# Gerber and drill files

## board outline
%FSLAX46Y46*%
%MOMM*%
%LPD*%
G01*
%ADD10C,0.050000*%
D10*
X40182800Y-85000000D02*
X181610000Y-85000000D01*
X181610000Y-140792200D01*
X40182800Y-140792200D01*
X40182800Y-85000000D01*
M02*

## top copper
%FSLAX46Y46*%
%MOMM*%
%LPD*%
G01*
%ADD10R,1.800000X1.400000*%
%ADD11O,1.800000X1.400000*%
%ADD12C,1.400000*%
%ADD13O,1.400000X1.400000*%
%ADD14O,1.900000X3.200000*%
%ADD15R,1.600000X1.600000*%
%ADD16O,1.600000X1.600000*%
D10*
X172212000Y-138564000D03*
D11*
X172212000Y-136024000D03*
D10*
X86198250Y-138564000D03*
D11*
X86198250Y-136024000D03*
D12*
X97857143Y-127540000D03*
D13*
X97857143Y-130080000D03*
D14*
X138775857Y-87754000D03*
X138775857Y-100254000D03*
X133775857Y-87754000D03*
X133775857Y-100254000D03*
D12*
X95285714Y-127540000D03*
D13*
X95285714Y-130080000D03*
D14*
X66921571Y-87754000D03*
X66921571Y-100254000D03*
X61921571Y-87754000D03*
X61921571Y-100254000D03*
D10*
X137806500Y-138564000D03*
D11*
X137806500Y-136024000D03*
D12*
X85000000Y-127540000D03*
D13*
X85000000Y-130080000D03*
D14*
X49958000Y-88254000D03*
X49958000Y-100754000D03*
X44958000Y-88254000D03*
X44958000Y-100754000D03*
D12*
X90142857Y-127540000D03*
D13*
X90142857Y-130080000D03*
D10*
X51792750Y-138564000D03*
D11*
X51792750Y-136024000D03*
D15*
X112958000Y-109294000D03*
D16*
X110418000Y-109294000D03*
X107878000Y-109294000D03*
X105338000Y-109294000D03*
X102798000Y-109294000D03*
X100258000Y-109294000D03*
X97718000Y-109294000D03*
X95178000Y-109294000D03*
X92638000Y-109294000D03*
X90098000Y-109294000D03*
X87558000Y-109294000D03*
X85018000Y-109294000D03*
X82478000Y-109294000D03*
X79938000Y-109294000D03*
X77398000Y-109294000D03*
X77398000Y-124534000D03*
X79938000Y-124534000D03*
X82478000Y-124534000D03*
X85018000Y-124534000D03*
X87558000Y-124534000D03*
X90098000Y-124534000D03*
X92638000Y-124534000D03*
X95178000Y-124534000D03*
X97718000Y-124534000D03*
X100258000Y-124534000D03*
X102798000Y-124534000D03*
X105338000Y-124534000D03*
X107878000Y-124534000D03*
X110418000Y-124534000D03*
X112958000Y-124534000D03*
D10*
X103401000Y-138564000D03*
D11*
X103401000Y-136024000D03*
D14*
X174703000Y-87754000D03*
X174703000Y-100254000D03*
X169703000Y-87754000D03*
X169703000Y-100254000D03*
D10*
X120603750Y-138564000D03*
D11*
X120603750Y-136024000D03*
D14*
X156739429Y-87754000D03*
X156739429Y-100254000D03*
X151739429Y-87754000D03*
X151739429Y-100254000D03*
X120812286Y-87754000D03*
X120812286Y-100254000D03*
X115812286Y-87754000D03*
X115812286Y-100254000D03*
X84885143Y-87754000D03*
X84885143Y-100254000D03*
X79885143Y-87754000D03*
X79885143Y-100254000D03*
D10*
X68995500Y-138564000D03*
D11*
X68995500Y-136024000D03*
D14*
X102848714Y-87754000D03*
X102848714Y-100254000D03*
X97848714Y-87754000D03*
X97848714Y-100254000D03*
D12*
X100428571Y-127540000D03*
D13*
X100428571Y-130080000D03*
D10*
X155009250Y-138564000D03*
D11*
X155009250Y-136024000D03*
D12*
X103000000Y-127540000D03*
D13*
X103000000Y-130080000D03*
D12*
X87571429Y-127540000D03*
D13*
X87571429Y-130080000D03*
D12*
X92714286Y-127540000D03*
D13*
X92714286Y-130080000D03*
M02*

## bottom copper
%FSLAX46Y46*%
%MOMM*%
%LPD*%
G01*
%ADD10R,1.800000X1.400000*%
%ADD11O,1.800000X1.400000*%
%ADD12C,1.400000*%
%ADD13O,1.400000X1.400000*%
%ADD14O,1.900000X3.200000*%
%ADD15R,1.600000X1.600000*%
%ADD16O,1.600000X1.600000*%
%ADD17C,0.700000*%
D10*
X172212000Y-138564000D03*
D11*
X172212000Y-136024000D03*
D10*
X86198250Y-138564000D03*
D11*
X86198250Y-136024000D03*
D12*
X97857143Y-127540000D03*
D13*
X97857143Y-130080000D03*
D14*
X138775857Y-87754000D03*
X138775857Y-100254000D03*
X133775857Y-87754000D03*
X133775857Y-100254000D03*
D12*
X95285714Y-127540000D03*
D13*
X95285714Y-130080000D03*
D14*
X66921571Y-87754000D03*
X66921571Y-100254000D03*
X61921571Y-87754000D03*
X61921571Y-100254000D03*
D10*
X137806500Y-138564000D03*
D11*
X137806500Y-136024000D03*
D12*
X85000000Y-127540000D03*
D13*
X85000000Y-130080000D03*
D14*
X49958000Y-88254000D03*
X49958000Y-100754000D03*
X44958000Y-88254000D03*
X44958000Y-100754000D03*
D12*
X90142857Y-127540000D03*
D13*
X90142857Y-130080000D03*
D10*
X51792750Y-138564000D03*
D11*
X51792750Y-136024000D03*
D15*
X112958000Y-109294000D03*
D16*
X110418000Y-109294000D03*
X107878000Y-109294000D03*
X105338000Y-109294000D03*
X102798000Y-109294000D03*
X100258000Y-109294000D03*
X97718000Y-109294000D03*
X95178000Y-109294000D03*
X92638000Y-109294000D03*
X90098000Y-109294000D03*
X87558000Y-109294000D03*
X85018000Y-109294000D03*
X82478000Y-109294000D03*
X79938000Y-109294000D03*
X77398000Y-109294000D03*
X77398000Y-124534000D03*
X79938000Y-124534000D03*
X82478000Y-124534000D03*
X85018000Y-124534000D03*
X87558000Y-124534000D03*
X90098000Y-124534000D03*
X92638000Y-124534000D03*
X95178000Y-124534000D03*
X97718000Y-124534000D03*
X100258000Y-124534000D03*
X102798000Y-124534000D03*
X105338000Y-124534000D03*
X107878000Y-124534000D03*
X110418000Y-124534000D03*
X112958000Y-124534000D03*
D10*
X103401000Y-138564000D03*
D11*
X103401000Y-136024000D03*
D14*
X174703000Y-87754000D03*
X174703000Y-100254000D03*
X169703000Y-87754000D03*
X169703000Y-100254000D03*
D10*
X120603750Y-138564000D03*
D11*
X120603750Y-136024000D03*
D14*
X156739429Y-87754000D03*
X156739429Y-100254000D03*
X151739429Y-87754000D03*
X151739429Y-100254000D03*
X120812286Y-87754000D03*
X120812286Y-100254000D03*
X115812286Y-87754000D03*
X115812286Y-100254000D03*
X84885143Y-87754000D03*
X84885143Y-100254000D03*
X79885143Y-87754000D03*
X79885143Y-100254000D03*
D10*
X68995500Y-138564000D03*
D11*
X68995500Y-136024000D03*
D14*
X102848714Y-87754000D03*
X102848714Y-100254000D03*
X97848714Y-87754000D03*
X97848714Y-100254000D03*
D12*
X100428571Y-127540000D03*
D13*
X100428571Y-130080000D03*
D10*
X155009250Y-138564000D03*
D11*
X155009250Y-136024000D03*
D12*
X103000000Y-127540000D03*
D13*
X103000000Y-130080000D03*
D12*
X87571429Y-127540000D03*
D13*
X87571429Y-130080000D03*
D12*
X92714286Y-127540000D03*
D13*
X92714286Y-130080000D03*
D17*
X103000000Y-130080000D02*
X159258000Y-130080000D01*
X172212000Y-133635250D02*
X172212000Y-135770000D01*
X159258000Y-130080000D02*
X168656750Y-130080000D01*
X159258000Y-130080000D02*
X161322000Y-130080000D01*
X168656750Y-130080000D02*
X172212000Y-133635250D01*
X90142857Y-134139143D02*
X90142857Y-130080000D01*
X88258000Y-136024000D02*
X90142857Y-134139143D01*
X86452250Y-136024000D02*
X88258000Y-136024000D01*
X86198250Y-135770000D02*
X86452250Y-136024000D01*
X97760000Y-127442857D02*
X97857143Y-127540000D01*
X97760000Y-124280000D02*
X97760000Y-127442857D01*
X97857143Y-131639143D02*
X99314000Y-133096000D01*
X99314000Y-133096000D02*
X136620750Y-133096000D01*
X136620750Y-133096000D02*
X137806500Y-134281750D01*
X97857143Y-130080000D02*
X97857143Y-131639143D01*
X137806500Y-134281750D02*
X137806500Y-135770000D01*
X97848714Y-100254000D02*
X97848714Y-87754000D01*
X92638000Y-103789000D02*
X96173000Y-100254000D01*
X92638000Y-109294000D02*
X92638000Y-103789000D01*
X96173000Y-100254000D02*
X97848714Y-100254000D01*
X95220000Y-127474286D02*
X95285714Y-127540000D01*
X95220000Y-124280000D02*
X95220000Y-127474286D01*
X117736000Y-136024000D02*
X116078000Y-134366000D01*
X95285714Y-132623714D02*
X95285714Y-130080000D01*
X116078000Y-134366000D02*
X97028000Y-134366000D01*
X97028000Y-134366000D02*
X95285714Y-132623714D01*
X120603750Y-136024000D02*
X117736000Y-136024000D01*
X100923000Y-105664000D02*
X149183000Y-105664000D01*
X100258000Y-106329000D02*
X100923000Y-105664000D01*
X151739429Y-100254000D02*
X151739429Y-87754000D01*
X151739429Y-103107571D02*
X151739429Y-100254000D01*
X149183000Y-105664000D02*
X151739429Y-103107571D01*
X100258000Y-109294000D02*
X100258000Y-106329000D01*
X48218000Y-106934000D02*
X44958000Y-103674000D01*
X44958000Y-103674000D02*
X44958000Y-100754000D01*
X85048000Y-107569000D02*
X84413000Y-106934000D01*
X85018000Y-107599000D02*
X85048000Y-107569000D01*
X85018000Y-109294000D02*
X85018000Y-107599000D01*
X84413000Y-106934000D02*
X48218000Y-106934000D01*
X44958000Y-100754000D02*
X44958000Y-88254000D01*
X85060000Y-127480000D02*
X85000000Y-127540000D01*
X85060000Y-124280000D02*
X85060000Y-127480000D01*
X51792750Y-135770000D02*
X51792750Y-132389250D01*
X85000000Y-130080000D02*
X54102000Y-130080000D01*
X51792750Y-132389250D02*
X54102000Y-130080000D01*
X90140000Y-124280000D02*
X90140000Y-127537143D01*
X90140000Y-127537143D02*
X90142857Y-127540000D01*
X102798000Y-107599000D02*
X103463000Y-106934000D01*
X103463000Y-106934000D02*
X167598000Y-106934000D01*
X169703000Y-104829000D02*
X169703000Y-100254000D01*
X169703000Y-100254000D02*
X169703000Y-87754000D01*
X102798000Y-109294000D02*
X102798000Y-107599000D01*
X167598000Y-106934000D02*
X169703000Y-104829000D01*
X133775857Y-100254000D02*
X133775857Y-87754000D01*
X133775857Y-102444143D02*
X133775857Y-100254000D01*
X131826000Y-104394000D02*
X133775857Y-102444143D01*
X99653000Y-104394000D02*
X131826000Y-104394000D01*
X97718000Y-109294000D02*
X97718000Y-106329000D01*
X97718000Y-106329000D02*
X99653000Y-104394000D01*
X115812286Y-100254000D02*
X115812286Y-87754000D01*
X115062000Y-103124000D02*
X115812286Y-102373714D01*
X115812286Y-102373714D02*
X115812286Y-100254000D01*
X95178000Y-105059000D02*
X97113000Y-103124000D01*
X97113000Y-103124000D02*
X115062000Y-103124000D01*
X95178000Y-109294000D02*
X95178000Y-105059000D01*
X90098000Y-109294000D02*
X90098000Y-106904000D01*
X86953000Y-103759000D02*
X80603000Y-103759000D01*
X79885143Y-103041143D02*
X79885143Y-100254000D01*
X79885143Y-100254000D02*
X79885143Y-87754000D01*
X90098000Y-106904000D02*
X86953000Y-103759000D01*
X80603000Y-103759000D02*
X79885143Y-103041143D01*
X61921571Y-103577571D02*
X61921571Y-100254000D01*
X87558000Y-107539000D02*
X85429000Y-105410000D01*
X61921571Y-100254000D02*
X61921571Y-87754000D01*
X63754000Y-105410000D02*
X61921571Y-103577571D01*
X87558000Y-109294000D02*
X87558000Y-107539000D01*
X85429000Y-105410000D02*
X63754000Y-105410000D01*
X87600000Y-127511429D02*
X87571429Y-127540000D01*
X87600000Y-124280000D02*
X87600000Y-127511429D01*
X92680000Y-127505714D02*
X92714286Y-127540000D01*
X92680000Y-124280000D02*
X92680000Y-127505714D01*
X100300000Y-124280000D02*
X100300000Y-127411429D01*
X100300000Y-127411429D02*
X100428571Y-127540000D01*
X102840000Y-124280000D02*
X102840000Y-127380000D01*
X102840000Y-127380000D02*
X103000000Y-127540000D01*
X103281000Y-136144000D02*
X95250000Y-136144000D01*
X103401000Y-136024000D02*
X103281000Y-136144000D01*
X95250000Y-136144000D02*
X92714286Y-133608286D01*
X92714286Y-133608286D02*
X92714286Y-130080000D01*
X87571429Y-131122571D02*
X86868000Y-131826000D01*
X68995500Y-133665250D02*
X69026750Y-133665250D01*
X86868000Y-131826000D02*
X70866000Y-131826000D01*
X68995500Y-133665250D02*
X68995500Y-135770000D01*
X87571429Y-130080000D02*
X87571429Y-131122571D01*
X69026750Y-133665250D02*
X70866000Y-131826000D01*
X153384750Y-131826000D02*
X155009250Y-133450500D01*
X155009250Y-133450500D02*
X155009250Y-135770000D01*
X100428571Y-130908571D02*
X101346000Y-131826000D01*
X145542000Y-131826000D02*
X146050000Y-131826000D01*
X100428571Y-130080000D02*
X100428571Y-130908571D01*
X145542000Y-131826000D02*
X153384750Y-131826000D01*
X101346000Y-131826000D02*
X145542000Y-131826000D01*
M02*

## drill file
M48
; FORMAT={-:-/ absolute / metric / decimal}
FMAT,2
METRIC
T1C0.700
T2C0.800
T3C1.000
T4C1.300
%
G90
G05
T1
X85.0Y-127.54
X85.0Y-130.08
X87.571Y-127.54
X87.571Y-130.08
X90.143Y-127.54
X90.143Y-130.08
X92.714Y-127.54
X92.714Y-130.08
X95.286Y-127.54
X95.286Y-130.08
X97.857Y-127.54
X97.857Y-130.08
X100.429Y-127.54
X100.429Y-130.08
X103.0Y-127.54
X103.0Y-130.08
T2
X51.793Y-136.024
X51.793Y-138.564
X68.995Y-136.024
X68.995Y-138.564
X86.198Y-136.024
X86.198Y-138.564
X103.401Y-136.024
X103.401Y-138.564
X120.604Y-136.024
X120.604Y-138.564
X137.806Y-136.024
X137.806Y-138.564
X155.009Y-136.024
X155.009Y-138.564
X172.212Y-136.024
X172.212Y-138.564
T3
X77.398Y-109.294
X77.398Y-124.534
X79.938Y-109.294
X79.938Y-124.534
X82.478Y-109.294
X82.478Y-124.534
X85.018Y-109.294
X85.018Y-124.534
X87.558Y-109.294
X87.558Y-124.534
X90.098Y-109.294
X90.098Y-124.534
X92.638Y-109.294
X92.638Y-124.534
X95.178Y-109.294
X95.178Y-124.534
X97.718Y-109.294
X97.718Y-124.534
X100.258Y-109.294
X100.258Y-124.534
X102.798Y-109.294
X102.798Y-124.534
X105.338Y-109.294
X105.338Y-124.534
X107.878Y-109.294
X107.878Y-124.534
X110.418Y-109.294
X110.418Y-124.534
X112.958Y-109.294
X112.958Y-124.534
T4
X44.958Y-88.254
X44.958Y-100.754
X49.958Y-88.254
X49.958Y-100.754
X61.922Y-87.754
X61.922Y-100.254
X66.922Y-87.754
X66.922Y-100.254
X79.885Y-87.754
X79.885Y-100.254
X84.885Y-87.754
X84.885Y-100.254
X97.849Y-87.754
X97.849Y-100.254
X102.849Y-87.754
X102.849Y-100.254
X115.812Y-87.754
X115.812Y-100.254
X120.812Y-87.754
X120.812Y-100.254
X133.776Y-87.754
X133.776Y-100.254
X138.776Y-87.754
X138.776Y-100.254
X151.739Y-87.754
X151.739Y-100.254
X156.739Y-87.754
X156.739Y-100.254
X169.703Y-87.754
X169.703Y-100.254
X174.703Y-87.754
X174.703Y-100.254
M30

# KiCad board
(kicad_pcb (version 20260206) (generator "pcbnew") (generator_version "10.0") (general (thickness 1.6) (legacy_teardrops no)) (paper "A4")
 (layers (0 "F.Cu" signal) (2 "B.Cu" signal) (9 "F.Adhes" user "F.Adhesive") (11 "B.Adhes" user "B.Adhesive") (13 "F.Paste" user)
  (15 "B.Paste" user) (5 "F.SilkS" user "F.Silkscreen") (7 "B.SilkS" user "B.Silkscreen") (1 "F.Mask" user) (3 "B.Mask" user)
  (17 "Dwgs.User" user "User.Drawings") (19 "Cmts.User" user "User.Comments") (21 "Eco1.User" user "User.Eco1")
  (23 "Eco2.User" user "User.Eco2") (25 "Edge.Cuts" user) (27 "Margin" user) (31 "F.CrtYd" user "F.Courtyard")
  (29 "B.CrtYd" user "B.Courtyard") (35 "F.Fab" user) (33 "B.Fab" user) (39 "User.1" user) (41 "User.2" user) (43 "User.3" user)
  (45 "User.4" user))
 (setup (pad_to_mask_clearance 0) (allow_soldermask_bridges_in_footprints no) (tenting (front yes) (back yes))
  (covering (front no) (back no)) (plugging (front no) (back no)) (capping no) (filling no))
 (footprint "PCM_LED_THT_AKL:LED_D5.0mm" (layer "F.Cu") (at 172.212 138.564 90)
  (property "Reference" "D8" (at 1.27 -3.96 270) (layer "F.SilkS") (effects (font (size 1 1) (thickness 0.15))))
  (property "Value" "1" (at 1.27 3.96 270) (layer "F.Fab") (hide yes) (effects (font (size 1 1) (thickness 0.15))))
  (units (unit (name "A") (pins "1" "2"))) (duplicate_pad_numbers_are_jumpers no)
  (pad "1" thru_hole rect (at 0 0 90) (size 1.4 1.8) (drill 0.8) (layers "*.Cu" "*.Mask") (remove_unused_layers no) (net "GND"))
  (pad "2" thru_hole oval (at 2.54 0 90) (size 1.4 1.8) (drill 0.8) (layers "*.Cu" "*.Mask") (remove_unused_layers no) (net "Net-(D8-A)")))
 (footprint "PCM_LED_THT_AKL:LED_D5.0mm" (layer "F.Cu") (at 86.19825 138.564 90)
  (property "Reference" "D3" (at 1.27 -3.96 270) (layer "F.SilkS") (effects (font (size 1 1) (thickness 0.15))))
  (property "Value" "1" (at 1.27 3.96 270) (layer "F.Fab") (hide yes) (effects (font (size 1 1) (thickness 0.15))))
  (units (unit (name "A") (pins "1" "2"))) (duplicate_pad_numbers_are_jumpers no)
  (pad "1" thru_hole rect (at 0 0 90) (size 1.4 1.8) (drill 0.8) (layers "*.Cu" "*.Mask") (remove_unused_layers no) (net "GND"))
  (pad "2" thru_hole oval (at 2.54 0 90) (size 1.4 1.8) (drill 0.8) (layers "*.Cu" "*.Mask") (remove_unused_layers no) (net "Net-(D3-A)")))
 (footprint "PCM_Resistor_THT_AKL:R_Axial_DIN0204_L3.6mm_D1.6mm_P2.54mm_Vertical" (layer "F.Cu") (at 97.857143 127.54 -90)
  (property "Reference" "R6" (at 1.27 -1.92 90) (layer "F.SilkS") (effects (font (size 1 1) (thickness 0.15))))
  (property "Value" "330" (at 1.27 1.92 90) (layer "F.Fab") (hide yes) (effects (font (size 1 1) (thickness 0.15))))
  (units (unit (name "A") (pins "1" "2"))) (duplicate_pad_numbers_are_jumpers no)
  (pad "1" thru_hole circle (at 0 0 270) (size 1.4 1.4) (drill 0.7) (layers "*.Cu" "*.Mask") (remove_unused_layers no) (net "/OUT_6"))
  (pad "2" thru_hole oval (at 2.54 0 270) (size 1.4 1.4) (drill 0.7) (layers "*.Cu" "*.Mask") (remove_unused_layers no) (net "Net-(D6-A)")))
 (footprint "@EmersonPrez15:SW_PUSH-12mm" (layer "F.Cu") (at 138.775857 87.754 -90)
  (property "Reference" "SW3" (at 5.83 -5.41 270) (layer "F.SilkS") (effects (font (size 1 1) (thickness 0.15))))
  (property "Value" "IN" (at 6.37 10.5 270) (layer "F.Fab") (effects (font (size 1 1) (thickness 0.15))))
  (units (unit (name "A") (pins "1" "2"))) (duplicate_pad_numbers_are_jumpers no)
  (pad "1" thru_hole oval (at 0 0 270) (size 3.2 1.9) (drill 1.3) (layers "*.Cu" "*.Mask") (remove_unused_layers no) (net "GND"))
  (pad "1" thru_hole oval (at 12.5 0 270) (size 3.2 1.9) (drill 1.3) (layers "*.Cu" "*.Mask") (remove_unused_layers no) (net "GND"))
  (pad "2" thru_hole oval (at 0 5 270) (size 3.2 1.9) (drill 1.3) (layers "*.Cu" "*.Mask") (remove_unused_layers no) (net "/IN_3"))
  (pad "2" thru_hole oval (at 12.5 5 270) (size 3.2 1.9) (drill 1.3) (layers "*.Cu" "*.Mask") (remove_unused_layers no) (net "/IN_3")))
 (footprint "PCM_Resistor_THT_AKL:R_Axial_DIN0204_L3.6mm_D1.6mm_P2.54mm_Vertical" (layer "F.Cu") (at 95.285714 127.54 -90)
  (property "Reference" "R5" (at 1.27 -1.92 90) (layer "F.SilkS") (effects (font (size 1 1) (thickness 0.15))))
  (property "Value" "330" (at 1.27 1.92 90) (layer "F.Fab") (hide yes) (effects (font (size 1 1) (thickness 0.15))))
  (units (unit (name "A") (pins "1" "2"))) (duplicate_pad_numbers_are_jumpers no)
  (pad "1" thru_hole circle (at 0 0 270) (size 1.4 1.4) (drill 0.7) (layers "*.Cu" "*.Mask") (remove_unused_layers no) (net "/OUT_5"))
  (pad "2" thru_hole oval (at 2.54 0 270) (size 1.4 1.4) (drill 0.7) (layers "*.Cu" "*.Mask") (remove_unused_layers no) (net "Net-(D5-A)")))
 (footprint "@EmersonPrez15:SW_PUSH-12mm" (layer "F.Cu") (at 66.921571 87.754 -90)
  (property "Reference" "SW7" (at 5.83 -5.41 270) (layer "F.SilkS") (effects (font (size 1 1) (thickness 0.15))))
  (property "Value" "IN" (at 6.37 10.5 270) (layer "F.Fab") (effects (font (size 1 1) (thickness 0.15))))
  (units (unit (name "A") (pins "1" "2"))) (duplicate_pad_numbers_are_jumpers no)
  (pad "1" thru_hole oval (at 0 0 270) (size 3.2 1.9) (drill 1.3) (layers "*.Cu" "*.Mask") (remove_unused_layers no) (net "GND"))
  (pad "1" thru_hole oval (at 12.5 0 270) (size 3.2 1.9) (drill 1.3) (layers "*.Cu" "*.Mask") (remove_unused_layers no) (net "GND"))
  (pad "2" thru_hole oval (at 0 5 270) (size 3.2 1.9) (drill 1.3) (layers "*.Cu" "*.Mask") (remove_unused_layers no) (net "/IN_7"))
  (pad "2" thru_hole oval (at 12.5 5 270) (size 3.2 1.9) (drill 1.3) (layers "*.Cu" "*.Mask") (remove_unused_layers no) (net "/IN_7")))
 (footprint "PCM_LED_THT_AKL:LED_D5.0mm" (layer "F.Cu") (at 137.8065 138.564 90)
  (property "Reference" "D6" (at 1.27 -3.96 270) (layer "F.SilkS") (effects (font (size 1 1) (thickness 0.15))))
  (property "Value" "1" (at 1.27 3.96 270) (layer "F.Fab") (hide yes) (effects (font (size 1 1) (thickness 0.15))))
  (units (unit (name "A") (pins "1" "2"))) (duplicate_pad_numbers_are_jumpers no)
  (pad "1" thru_hole rect (at 0 0 90) (size 1.4 1.8) (drill 0.8) (layers "*.Cu" "*.Mask") (remove_unused_layers no) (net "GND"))
  (pad "2" thru_hole oval (at 2.54 0 90) (size 1.4 1.8) (drill 0.8) (layers "*.Cu" "*.Mask") (remove_unused_layers no) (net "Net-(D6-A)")))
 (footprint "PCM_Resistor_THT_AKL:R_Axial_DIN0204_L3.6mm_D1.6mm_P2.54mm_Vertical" (layer "F.Cu") (at 85 127.54 -90)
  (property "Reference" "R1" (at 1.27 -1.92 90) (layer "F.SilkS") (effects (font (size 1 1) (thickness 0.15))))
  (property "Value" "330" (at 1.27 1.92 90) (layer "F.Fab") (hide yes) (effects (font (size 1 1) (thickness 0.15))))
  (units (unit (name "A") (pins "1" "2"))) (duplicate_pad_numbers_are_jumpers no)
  (pad "1" thru_hole circle (at 0 0 270) (size 1.4 1.4) (drill 0.7) (layers "*.Cu" "*.Mask") (remove_unused_layers no) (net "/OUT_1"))
  (pad "2" thru_hole oval (at 2.54 0 270) (size 1.4 1.4) (drill 0.7) (layers "*.Cu" "*.Mask") (remove_unused_layers no) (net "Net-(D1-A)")))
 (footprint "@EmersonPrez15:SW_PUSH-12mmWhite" (layer "F.Cu") (at 49.958 88.254 -90)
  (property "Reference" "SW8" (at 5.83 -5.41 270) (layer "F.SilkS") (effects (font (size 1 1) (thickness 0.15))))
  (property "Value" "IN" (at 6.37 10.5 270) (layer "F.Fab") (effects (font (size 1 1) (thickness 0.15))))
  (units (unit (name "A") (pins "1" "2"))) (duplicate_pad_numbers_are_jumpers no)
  (pad "1" thru_hole oval (at 0 0 270) (size 3.2 1.9) (drill 1.3) (layers "*.Cu" "*.Mask") (remove_unused_layers no) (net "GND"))
  (pad "1" thru_hole oval (at 12.5 0 270) (size 3.2 1.9) (drill 1.3) (layers "*.Cu" "*.Mask") (remove_unused_layers no) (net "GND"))
  (pad "2" thru_hole oval (at 0 5 270) (size 3.2 1.9) (drill 1.3) (layers "*.Cu" "*.Mask") (remove_unused_layers no) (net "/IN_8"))
  (pad "2" thru_hole oval (at 12.5 5 270) (size 3.2 1.9) (drill 1.3) (layers "*.Cu" "*.Mask") (remove_unused_layers no) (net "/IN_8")))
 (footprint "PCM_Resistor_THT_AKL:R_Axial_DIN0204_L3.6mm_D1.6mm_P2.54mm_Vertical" (layer "F.Cu") (at 90.142857 127.54 -90)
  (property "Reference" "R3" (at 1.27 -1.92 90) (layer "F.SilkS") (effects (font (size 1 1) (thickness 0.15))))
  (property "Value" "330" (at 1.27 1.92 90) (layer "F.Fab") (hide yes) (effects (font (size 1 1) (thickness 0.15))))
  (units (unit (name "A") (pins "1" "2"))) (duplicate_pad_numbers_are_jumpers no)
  (pad "1" thru_hole circle (at 0 0 270) (size 1.4 1.4) (drill 0.7) (layers "*.Cu" "*.Mask") (remove_unused_layers no) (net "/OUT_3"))
  (pad "2" thru_hole oval (at 2.54 0 270) (size 1.4 1.4) (drill 0.7) (layers "*.Cu" "*.Mask") (remove_unused_layers no) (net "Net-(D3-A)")))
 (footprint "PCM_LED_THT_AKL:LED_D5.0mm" (layer "F.Cu") (at 51.79275 138.564 90)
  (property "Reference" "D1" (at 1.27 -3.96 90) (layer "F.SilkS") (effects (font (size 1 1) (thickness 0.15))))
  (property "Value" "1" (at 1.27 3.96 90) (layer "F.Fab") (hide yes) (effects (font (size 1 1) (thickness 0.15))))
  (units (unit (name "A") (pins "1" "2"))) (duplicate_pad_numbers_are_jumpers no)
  (pad "1" thru_hole rect (at 0 0 90) (size 1.4 1.8) (drill 0.8) (layers "*.Cu" "*.Mask") (remove_unused_layers no) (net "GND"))
  (pad "2" thru_hole oval (at 2.54 0 90) (size 1.4 1.8) (drill 0.8) (layers "*.Cu" "*.Mask") (remove_unused_layers no) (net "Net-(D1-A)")))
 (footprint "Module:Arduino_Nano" (layer "F.Cu") (at 112.958 109.294 -90)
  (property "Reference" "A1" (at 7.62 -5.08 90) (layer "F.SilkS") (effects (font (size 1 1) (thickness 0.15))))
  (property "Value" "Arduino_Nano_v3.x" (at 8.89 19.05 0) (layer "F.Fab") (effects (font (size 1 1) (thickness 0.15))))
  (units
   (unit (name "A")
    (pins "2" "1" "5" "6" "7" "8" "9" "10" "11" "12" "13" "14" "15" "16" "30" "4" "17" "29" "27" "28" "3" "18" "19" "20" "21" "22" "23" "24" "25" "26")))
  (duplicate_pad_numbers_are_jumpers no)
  (pad "1" thru_hole rect (at 0 0 270) (size 1.6 1.6) (drill 1) (layers "*.Cu" "*.Mask") (remove_unused_layers no)
   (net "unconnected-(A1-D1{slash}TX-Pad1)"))
  (pad "2" thru_hole oval (at 0 2.54 270) (size 1.6 1.6) (drill 1) (layers "*.Cu" "*.Mask") (remove_unused_layers no)
   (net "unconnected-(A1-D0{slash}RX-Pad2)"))
  (pad "3" thru_hole oval (at 0 5.08 270) (size 1.6 1.6) (drill 1) (layers "*.Cu" "*.Mask") (remove_unused_layers no)
   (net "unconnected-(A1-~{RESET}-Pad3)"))
  (pad "4" thru_hole oval (at 0 7.62 270) (size 1.6 1.6) (drill 1) (layers "*.Cu" "*.Mask") (remove_unused_layers no) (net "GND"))
  (pad "5" thru_hole oval (at 0 10.16 270) (size 1.6 1.6) (drill 1) (layers "*.Cu" "*.Mask") (remove_unused_layers no) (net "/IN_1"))
  (pad "6" thru_hole oval (at 0 12.7 270) (size 1.6 1.6) (drill 1) (layers "*.Cu" "*.Mask") (remove_unused_layers no) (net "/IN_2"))
  (pad "7" thru_hole oval (at 0 15.24 270) (size 1.6 1.6) (drill 1) (layers "*.Cu" "*.Mask") (remove_unused_layers no) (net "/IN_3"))
  (pad "8" thru_hole oval (at 0 17.78 270) (size 1.6 1.6) (drill 1) (layers "*.Cu" "*.Mask") (remove_unused_layers no) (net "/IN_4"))
  (pad "9" thru_hole oval (at 0 20.32 270) (size 1.6 1.6) (drill 1) (layers "*.Cu" "*.Mask") (remove_unused_layers no) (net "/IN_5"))
  (pad "10" thru_hole oval (at 0 22.86 270) (size 1.6 1.6) (drill 1) (layers "*.Cu" "*.Mask") (remove_unused_layers no) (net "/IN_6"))
  (pad "11" thru_hole oval (at 0 25.4 270) (size 1.6 1.6) (drill 1) (layers "*.Cu" "*.Mask") (remove_unused_layers no) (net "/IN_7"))
  (pad "12" thru_hole oval (at 0 27.94 270) (size 1.6 1.6) (drill 1) (layers "*.Cu" "*.Mask") (remove_unused_layers no) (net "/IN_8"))
  (pad "13" thru_hole oval (at 0 30.48 270) (size 1.6 1.6) (drill 1) (layers "*.Cu" "*.Mask") (remove_unused_layers no) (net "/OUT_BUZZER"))
  (pad "14" thru_hole oval (at 0 33.02 270) (size 1.6 1.6) (drill 1) (layers "*.Cu" "*.Mask") (remove_unused_layers no)
   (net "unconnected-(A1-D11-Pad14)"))
  (pad "15" thru_hole oval (at 0 35.56 270) (size 1.6 1.6) (drill 1) (layers "*.Cu" "*.Mask") (remove_unused_layers no)
   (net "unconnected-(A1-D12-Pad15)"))
  (pad "16" thru_hole oval (at 15.24 35.56 270) (size 1.6 1.6) (drill 1) (layers "*.Cu" "*.Mask") (remove_unused_layers no)
   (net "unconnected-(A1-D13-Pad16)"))
  (pad "17" thru_hole oval (at 15.24 33.02 270) (size 1.6 1.6) (drill 1) (layers "*.Cu" "*.Mask") (remove_unused_layers no)
   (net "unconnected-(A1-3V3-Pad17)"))
  (pad "18" thru_hole oval (at 15.24 30.48 270) (size 1.6 1.6) (drill 1) (layers "*.Cu" "*.Mask") (remove_unused_layers no)
   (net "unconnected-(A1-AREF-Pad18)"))
  (pad "19" thru_hole oval (at 15.24 27.94 270) (size 1.6 1.6) (drill 1) (layers "*.Cu" "*.Mask") (remove_unused_layers no) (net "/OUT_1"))
  (pad "20" thru_hole oval (at 15.24 25.4 270) (size 1.6 1.6) (drill 1) (layers "*.Cu" "*.Mask") (remove_unused_layers no) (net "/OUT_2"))
  (pad "21" thru_hole oval (at 15.24 22.86 270) (size 1.6 1.6) (drill 1) (layers "*.Cu" "*.Mask") (remove_unused_layers no) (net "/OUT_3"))
  (pad "22" thru_hole oval (at 15.24 20.32 270) (size 1.6 1.6) (drill 1) (layers "*.Cu" "*.Mask") (remove_unused_layers no) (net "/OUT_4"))
  (pad "23" thru_hole oval (at 15.24 17.78 270) (size 1.6 1.6) (drill 1) (layers "*.Cu" "*.Mask") (remove_unused_layers no) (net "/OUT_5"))
  (pad "24" thru_hole oval (at 15.24 15.24 270) (size 1.6 1.6) (drill 1) (layers "*.Cu" "*.Mask") (remove_unused_layers no) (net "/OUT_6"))
  (pad "25" thru_hole oval (at 15.24 12.7 270) (size 1.6 1.6) (drill 1) (layers "*.Cu" "*.Mask") (remove_unused_layers no) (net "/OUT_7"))
  (pad "26" thru_hole oval (at 15.24 10.16 270) (size 1.6 1.6) (drill 1) (layers "*.Cu" "*.Mask") (remove_unused_layers no) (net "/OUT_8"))
  (pad "27" thru_hole oval (at 15.24 7.62 270) (size 1.6 1.6) (drill 1) (layers "*.Cu" "*.Mask") (remove_unused_layers no) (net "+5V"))
  (pad "28" thru_hole oval (at 15.24 5.08 270) (size 1.6 1.6) (drill 1) (layers "*.Cu" "*.Mask") (remove_unused_layers no)
   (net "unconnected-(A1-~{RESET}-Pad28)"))
  (pad "29" thru_hole oval (at 15.24 2.54 270) (size 1.6 1.6) (drill 1) (layers "*.Cu" "*.Mask") (remove_unused_layers no) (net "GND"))
  (pad "30" thru_hole oval (at 15.24 0 270) (size 1.6 1.6) (drill 1) (layers "*.Cu" "*.Mask") (remove_unused_layers no)
   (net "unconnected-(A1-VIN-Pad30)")))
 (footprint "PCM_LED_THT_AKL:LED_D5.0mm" (layer "F.Cu") (at 103.401 138.564 90)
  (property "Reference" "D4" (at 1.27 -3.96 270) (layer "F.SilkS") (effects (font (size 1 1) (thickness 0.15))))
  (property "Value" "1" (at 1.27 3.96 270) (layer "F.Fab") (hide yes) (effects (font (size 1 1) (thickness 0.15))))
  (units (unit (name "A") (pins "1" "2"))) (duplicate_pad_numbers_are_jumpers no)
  (pad "1" thru_hole rect (at 0 0 90) (size 1.4 1.8) (drill 0.8) (layers "*.Cu" "*.Mask") (remove_unused_layers no) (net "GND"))
  (pad "2" thru_hole oval (at 2.54 0 90) (size 1.4 1.8) (drill 0.8) (layers "*.Cu" "*.Mask") (remove_unused_layers no) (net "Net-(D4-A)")))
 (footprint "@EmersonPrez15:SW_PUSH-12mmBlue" (layer "F.Cu") (at 174.703 87.754 -90)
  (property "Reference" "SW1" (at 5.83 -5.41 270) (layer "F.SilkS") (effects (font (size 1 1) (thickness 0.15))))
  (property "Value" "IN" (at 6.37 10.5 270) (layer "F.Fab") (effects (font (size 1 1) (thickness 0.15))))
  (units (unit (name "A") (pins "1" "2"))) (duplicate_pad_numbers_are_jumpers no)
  (pad "1" thru_hole oval (at 0 0 270) (size 3.2 1.9) (drill 1.3) (layers "*.Cu" "*.Mask") (remove_unused_layers no) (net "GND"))
  (pad "1" thru_hole oval (at 12.5 0 270) (size 3.2 1.9) (drill 1.3) (layers "*.Cu" "*.Mask") (remove_unused_layers no) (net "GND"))
  (pad "2" thru_hole oval (at 0 5 270) (size 3.2 1.9) (drill 1.3) (layers "*.Cu" "*.Mask") (remove_unused_layers no) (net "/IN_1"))
  (pad "2" thru_hole oval (at 12.5 5 270) (size 3.2 1.9) (drill 1.3) (layers "*.Cu" "*.Mask") (remove_unused_layers no) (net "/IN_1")))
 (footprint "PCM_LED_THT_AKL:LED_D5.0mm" (layer "F.Cu") (at 120.60375 138.564 90)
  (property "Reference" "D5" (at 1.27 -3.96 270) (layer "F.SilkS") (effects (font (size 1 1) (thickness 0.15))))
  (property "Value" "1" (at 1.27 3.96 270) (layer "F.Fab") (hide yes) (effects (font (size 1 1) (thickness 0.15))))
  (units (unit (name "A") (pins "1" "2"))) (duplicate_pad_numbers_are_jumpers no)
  (pad "1" thru_hole rect (at 0 0 90) (size 1.4 1.8) (drill 0.8) (layers "*.Cu" "*.Mask") (remove_unused_layers no) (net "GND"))
  (pad "2" thru_hole oval (at 2.54 0 90) (size 1.4 1.8) (drill 0.8) (layers "*.Cu" "*.Mask") (remove_unused_layers no) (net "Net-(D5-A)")))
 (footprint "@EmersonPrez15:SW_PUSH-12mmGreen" (layer "F.Cu") (at 156.739429 87.754 -90)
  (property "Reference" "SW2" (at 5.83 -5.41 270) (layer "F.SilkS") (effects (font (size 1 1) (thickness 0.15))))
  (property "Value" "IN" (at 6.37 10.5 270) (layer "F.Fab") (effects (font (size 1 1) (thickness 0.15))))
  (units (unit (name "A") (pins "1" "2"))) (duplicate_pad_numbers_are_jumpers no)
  (pad "1" thru_hole oval (at 0 0 270) (size 3.2 1.9) (drill 1.3) (layers "*.Cu" "*.Mask") (remove_unused_layers no) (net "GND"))
  (pad "1" thru_hole oval (at 12.5 0 270) (size 3.2 1.9) (drill 1.3) (layers "*.Cu" "*.Mask") (remove_unused_layers no) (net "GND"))
  (pad "2" thru_hole oval (at 0 5 270) (size 3.2 1.9) (drill 1.3) (layers "*.Cu" "*.Mask") (remove_unused_layers no) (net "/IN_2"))
  (pad "2" thru_hole oval (at 12.5 5 270) (size 3.2 1.9) (drill 1.3) (layers "*.Cu" "*.Mask") (remove_unused_layers no) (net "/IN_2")))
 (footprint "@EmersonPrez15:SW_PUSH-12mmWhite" (layer "F.Cu") (at 120.812286 87.754 -90)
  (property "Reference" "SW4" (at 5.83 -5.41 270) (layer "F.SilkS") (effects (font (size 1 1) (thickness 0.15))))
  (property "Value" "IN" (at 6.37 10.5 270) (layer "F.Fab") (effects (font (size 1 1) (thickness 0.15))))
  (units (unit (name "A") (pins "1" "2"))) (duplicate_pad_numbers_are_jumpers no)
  (pad "1" thru_hole oval (at 0 0 270) (size 3.2 1.9) (drill 1.3) (layers "*.Cu" "*.Mask") (remove_unused_layers no) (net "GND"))
  (pad "1" thru_hole oval (at 12.5 0 270) (size 3.2 1.9) (drill 1.3) (layers "*.Cu" "*.Mask") (remove_unused_layers no) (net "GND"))
  (pad "2" thru_hole oval (at 0 5 270) (size 3.2 1.9) (drill 1.3) (layers "*.Cu" "*.Mask") (remove_unused_layers no) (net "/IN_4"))
  (pad "2" thru_hole oval (at 12.5 5 270) (size 3.2 1.9) (drill 1.3) (layers "*.Cu" "*.Mask") (remove_unused_layers no) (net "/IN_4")))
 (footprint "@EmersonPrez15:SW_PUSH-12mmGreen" (layer "F.Cu") (at 84.885143 87.754 -90)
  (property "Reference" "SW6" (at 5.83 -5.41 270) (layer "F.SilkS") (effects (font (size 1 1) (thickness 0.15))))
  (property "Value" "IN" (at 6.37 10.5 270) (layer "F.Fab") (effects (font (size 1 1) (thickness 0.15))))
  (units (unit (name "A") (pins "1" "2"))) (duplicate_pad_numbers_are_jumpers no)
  (pad "1" thru_hole oval (at 0 0 270) (size 3.2 1.9) (drill 1.3) (layers "*.Cu" "*.Mask") (remove_unused_layers no) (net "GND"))
  (pad "1" thru_hole oval (at 12.5 0 270) (size 3.2 1.9) (drill 1.3) (layers "*.Cu" "*.Mask") (remove_unused_layers no) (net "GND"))
  (pad "2" thru_hole oval (at 0 5 270) (size 3.2 1.9) (drill 1.3) (layers "*.Cu" "*.Mask") (remove_unused_layers no) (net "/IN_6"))
  (pad "2" thru_hole oval (at 12.5 5 270) (size 3.2 1.9) (drill 1.3) (layers "*.Cu" "*.Mask") (remove_unused_layers no) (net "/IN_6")))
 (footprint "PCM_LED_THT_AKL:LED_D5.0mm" (layer "F.Cu") (at 68.9955 138.564 90)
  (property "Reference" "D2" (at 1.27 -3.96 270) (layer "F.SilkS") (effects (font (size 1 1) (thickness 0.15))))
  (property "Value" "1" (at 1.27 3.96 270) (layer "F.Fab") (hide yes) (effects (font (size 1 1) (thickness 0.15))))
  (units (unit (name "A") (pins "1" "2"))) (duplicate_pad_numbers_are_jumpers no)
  (pad "1" thru_hole rect (at 0 0 90) (size 1.4 1.8) (drill 0.8) (layers "*.Cu" "*.Mask") (remove_unused_layers no) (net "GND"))
  (pad "2" thru_hole oval (at 2.54 0 90) (size 1.4 1.8) (drill 0.8) (layers "*.Cu" "*.Mask") (remove_unused_layers no) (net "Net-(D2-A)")))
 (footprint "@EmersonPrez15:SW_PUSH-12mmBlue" (layer "F.Cu") (at 102.848714 87.754 -90)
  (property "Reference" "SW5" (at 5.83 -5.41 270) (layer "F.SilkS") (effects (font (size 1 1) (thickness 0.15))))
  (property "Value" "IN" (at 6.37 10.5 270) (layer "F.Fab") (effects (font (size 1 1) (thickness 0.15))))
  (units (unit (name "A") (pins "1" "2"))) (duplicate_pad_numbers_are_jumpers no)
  (pad "1" thru_hole oval (at 0 0 270) (size 3.2 1.9) (drill 1.3) (layers "*.Cu" "*.Mask") (remove_unused_layers no) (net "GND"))
  (pad "1" thru_hole oval (at 12.5 0 270) (size 3.2 1.9) (drill 1.3) (layers "*.Cu" "*.Mask") (remove_unused_layers no) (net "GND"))
  (pad "2" thru_hole oval (at 0 5 270) (size 3.2 1.9) (drill 1.3) (layers "*.Cu" "*.Mask") (remove_unused_layers no) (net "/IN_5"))
  (pad "2" thru_hole oval (at 12.5 5 270) (size 3.2 1.9) (drill 1.3) (layers "*.Cu" "*.Mask") (remove_unused_layers no) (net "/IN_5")))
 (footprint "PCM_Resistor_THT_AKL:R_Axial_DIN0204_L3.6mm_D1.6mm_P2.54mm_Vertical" (layer "F.Cu") (at 100.428571 127.54 -90)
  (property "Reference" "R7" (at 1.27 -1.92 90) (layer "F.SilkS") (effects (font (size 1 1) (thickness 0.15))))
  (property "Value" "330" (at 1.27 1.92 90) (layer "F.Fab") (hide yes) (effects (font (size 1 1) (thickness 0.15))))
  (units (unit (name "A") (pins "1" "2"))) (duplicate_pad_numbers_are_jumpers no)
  (pad "1" thru_hole circle (at 0 0 270) (size 1.4 1.4) (drill 0.7) (layers "*.Cu" "*.Mask") (remove_unused_layers no) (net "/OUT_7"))
  (pad "2" thru_hole oval (at 2.54 0 270) (size 1.4 1.4) (drill 0.7) (layers "*.Cu" "*.Mask") (remove_unused_layers no) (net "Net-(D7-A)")))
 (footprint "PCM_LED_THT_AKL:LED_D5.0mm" (layer "F.Cu") (at 155.00925 138.564 90)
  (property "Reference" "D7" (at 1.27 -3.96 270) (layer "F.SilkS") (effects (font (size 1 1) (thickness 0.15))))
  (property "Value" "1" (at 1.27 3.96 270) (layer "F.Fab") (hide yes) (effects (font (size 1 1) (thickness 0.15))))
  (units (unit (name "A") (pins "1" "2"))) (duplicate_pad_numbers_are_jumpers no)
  (pad "1" thru_hole rect (at 0 0 90) (size 1.4 1.8) (drill 0.8) (layers "*.Cu" "*.Mask") (remove_unused_layers no) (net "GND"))
  (pad "2" thru_hole oval (at 2.54 0 90) (size 1.4 1.8) (drill 0.8) (layers "*.Cu" "*.Mask") (remove_unused_layers no) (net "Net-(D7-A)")))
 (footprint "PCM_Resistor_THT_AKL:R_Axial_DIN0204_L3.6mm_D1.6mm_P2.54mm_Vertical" (layer "F.Cu") (at 103 127.54 -90)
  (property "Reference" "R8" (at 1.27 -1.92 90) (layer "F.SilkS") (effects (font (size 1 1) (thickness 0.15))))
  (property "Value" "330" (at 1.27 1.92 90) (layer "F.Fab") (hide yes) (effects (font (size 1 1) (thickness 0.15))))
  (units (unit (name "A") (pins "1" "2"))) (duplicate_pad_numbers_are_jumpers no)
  (pad "1" thru_hole circle (at 0 0 270) (size 1.4 1.4) (drill 0.7) (layers "*.Cu" "*.Mask") (remove_unused_layers no) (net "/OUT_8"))
  (pad "2" thru_hole oval (at 2.54 0 270) (size 1.4 1.4) (drill 0.7) (layers "*.Cu" "*.Mask") (remove_unused_layers no) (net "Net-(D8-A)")))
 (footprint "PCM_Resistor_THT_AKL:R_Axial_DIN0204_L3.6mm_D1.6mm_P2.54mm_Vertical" (layer "F.Cu") (at 87.571429 127.54 -90)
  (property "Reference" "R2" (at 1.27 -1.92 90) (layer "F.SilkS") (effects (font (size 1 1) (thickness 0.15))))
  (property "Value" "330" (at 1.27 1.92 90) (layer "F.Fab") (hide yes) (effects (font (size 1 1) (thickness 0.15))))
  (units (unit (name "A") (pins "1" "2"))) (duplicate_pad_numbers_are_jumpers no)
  (pad "1" thru_hole circle (at 0 0 270) (size 1.4 1.4) (drill 0.7) (layers "*.Cu" "*.Mask") (remove_unused_layers no) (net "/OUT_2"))
  (pad "2" thru_hole oval (at 2.54 0 270) (size 1.4 1.4) (drill 0.7) (layers "*.Cu" "*.Mask") (remove_unused_layers no) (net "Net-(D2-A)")))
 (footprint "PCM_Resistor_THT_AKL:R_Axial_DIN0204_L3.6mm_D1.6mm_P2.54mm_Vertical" (layer "F.Cu") (at 92.714286 127.54 -90)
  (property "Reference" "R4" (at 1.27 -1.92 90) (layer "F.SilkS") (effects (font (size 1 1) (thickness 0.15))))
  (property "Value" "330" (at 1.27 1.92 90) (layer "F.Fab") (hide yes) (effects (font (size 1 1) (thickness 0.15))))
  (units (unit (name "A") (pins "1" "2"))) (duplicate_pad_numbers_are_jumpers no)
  (pad "1" thru_hole circle (at 0 0 270) (size 1.4 1.4) (drill 0.7) (layers "*.Cu" "*.Mask") (remove_unused_layers no) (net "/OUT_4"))
  (pad "2" thru_hole oval (at 2.54 0 270) (size 1.4 1.4) (drill 0.7) (layers "*.Cu" "*.Mask") (remove_unused_layers no) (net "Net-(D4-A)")))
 (gr_rect (start 40.1828 85) (end 181.61 140.7922) (stroke (width 0.05) (type default)) (fill no) (layer "Edge.Cuts"))
 (segment (start 103 130.08) (end 159.258 130.08) (width 0.7) (layer "B.Cu") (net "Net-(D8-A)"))
 (segment (start 172.212 133.63525) (end 172.212 135.77) (width 0.7) (layer "B.Cu") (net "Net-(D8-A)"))
 (segment (start 159.258 130.08) (end 168.65675 130.08) (width 0.7) (layer "B.Cu") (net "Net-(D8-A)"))
 (segment (start 159.258 130.08) (end 161.322 130.08) (width 0.7) (layer "B.Cu") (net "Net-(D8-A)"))
 (segment (start 168.65675 130.08) (end 172.212 133.63525) (width 0.7) (layer "B.Cu") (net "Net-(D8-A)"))
 (segment (start 90.142857 134.139143) (end 90.142857 130.08) (width 0.7) (layer "B.Cu") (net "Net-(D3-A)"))
 (segment (start 88.258 136.024) (end 90.142857 134.139143) (width 0.7) (layer "B.Cu") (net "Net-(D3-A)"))
 (segment (start 86.45225 136.024) (end 88.258 136.024) (width 0.7) (layer "B.Cu") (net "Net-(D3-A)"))
 (segment (start 86.19825 135.77) (end 86.45225 136.024) (width 0.7) (layer "B.Cu") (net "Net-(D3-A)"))
 (segment (start 97.76 127.442857) (end 97.857143 127.54) (width 0.7) (layer "B.Cu") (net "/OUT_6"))
 (segment (start 97.76 124.28) (end 97.76 127.442857) (width 0.7) (layer "B.Cu") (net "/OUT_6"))
 (segment (start 97.857143 131.639143) (end 99.314 133.096) (width 0.7) (layer "B.Cu") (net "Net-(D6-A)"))
 (segment (start 99.314 133.096) (end 136.62075 133.096) (width 0.7) (layer "B.Cu") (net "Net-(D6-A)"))
 (segment (start 136.62075 133.096) (end 137.8065 134.28175) (width 0.7) (layer "B.Cu") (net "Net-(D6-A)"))
 (segment (start 97.857143 130.08) (end 97.857143 131.639143) (width 0.7) (layer "B.Cu") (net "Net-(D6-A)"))
 (segment (start 137.8065 134.28175) (end 137.8065 135.77) (width 0.7) (layer "B.Cu") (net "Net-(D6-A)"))
 (segment (start 97.848714 100.254) (end 97.848714 87.754) (width 0.7) (layer "B.Cu") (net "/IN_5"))
 (segment (start 92.638 103.789) (end 96.173 100.254) (width 0.7) (layer "B.Cu") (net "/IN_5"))
 (segment (start 92.638 109.294) (end 92.638 103.789) (width 0.7) (layer "B.Cu") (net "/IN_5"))
 (segment (start 96.173 100.254) (end 97.848714 100.254) (width 0.7) (layer "B.Cu") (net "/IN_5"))
 (segment (start 95.22 127.474286) (end 95.285714 127.54) (width 0.7) (layer "B.Cu") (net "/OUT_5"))
 (segment (start 95.22 124.28) (end 95.22 127.474286) (width 0.7) (layer "B.Cu") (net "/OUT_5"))
 (segment (start 117.736 136.024) (end 116.078 134.366) (width 0.7) (layer "B.Cu") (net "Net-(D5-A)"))
 (segment (start 95.285714 132.623714) (end 95.285714 130.08) (width 0.7) (layer "B.Cu") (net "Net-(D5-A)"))
 (segment (start 116.078 134.366) (end 97.028 134.366) (width 0.7) (layer "B.Cu") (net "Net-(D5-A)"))
 (segment (start 97.028 134.366) (end 95.285714 132.623714) (width 0.7) (layer "B.Cu") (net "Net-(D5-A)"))
 (segment (start 120.60375 136.024) (end 117.736 136.024) (width 0.7) (layer "B.Cu") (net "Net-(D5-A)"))
 (segment (start 100.923 105.664) (end 149.183 105.664) (width 0.7) (layer "B.Cu") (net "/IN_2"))
 (segment (start 100.258 106.329) (end 100.923 105.664) (width 0.7) (layer "B.Cu") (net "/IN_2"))
 (segment (start 151.739429 100.254) (end 151.739429 87.754) (width 0.7) (layer "B.Cu") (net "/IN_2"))
 (segment (start 151.739429 103.107571) (end 151.739429 100.254) (width 0.7) (layer "B.Cu") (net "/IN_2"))
 (segment (start 149.183 105.664) (end 151.739429 103.107571) (width 0.7) (layer "B.Cu") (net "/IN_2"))
 (segment (start 100.258 109.294) (end 100.258 106.329) (width 0.7) (layer "B.Cu") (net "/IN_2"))
 (segment (start 48.218 106.934) (end 44.958 103.674) (width 0.7) (layer "B.Cu") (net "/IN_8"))
 (segment (start 44.958 103.674) (end 44.958 100.754) (width 0.7) (layer "B.Cu") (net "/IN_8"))
 (segment (start 85.048 107.569) (end 84.413 106.934) (width 0.7) (layer "B.Cu") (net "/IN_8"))
 (segment (start 85.018 107.599) (end 85.048 107.569) (width 0.7) (layer "B.Cu") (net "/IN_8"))
 (segment (start 85.018 109.294) (end 85.018 107.599) (width 0.7) (layer "B.Cu") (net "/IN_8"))
 (segment (start 84.413 106.934) (end 48.218 106.934) (width 0.7) (layer "B.Cu") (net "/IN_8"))
 (segment (start 44.958 100.754) (end 44.958 88.254) (width 0.7) (layer "B.Cu") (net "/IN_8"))
 (segment (start 85.06 127.48) (end 85 127.54) (width 0.7) (layer "B.Cu") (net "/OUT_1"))
 (segment (start 85.06 124.28) (end 85.06 127.48) (width 0.7) (layer "B.Cu") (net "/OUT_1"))
 (segment (start 51.79275 135.77) (end 51.79275 132.38925) (width 0.7) (layer "B.Cu") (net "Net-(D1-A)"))
 (segment (start 85 130.08) (end 54.102 130.08) (width 0.7) (layer "B.Cu") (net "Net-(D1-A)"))
 (segment (start 51.79275 132.38925) (end 54.102 130.08) (width 0.7) (layer "B.Cu") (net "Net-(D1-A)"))
 (segment (start 90.14 124.28) (end 90.14 127.537143) (width 0.7) (layer "B.Cu") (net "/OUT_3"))
 (segment (start 90.14 127.537143) (end 90.142857 127.54) (width 0.7) (layer "B.Cu") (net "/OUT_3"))
 (segment (start 102.798 107.599) (end 103.463 106.934) (width 0.7) (layer "B.Cu") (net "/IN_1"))
 (segment (start 103.463 106.934) (end 167.598 106.934) (width 0.7) (layer "B.Cu") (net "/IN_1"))
 (segment (start 169.703 104.829) (end 169.703 100.254) (width 0.7) (layer "B.Cu") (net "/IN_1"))
 (segment (start 169.703 100.254) (end 169.703 87.754) (width 0.7) (layer "B.Cu") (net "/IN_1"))
 (segment (start 102.798 109.294) (end 102.798 107.599) (width 0.7) (layer "B.Cu") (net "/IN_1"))
 (segment (start 167.598 106.934) (end 169.703 104.829) (width 0.7) (layer "B.Cu") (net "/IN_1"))
 (segment (start 133.775857 100.254) (end 133.775857 87.754) (width 0.7) (layer "B.Cu") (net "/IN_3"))
 (segment (start 133.775857 102.444143) (end 133.775857 100.254) (width 0.7) (layer "B.Cu") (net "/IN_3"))
 (segment (start 131.826 104.394) (end 133.775857 102.444143) (width 0.7) (layer "B.Cu") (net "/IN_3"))
 (segment (start 99.653 104.394) (end 131.826 104.394) (width 0.7) (layer "B.Cu") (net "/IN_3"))
 (segment (start 97.718 109.294) (end 97.718 106.329) (width 0.7) (layer "B.Cu") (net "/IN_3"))
 (segment (start 97.718 106.329) (end 99.653 104.394) (width 0.7) (layer "B.Cu") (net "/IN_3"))
 (segment (start 115.812286 100.254) (end 115.812286 87.754) (width 0.7) (layer "B.Cu") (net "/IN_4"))
 (segment (start 115.062 103.124) (end 115.812286 102.373714) (width 0.7) (layer "B.Cu") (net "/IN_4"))
 (segment (start 115.812286 102.373714) (end 115.812286 100.254) (width 0.7) (layer "B.Cu") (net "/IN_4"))
 (segment (start 95.178 105.059) (end 97.113 103.124) (width 0.7) (layer "B.Cu") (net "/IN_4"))
 (segment (start 97.113 103.124) (end 115.062 103.124) (width 0.7) (layer "B.Cu") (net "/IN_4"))
 (segment (start 95.178 109.294) (end 95.178 105.059) (width 0.7) (layer "B.Cu") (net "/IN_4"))
 (segment (start 90.098 109.294) (end 90.098 106.904) (width 0.7) (layer "B.Cu") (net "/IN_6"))
 (segment (start 86.953 103.759) (end 80.603 103.759) (width 0.7) (layer "B.Cu") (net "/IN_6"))
 (segment (start 79.885143 103.041143) (end 79.885143 100.254) (width 0.7) (layer "B.Cu") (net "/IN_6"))
 (segment (start 79.885143 100.254) (end 79.885143 87.754) (width 0.7) (layer "B.Cu") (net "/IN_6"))
 (segment (start 90.098 106.904) (end 86.953 103.759) (width 0.7) (layer "B.Cu") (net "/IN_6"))
 (segment (start 80.603 103.759) (end 79.885143 103.041143) (width 0.7) (layer "B.Cu") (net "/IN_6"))
 (segment (start 61.921571 103.577571) (end 61.921571 100.254) (width 0.7) (layer "B.Cu") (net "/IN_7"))
 (segment (start 87.558 107.539) (end 85.429 105.41) (width 0.7) (layer "B.Cu") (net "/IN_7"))
 (segment (start 61.921571 100.254) (end 61.921571 87.754) (width 0.7) (layer "B.Cu") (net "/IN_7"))
 (segment (start 63.754 105.41) (end 61.921571 103.577571) (width 0.7) (layer "B.Cu") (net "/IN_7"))
 (segment (start 87.558 109.294) (end 87.558 107.539) (width 0.7) (layer "B.Cu") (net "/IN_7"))
 (segment (start 85.429 105.41) (end 63.754 105.41) (width 0.7) (layer "B.Cu") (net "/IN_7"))
 (segment (start 87.6 127.511429) (end 87.571429 127.54) (width 0.7) (layer "B.Cu") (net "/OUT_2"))
 (segment (start 87.6 124.28) (end 87.6 127.511429) (width 0.7) (layer "B.Cu") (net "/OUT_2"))
 (segment (start 92.68 127.505714) (end 92.714286 127.54) (width 0.7) (layer "B.Cu") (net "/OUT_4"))
 (segment (start 92.68 124.28) (end 92.68 127.505714) (width 0.7) (layer "B.Cu") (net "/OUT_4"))
 (segment (start 100.3 124.28) (end 100.3 127.411429) (width 0.7) (layer "B.Cu") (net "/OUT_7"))
 (segment (start 100.3 127.411429) (end 100.428571 127.54) (width 0.7) (layer "B.Cu") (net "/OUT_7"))
 (segment (start 102.84 124.28) (end 102.84 127.38) (width 0.7) (layer "B.Cu") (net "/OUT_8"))
 (segment (start 102.84 127.38) (end 103 127.54) (width 0.7) (layer "B.Cu") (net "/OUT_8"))
 (segment (start 103.281 136.144) (end 95.25 136.144) (width 0.7) (layer "B.Cu") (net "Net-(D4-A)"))
 (segment (start 103.401 136.024) (end 103.281 136.144) (width 0.7) (layer "B.Cu") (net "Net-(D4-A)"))
 (segment (start 95.25 136.144) (end 92.714286 133.608286) (width 0.7) (layer "B.Cu") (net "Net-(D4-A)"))
 (segment (start 92.714286 133.608286) (end 92.714286 130.08) (width 0.7) (layer "B.Cu") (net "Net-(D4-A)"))
 (segment (start 87.571429 131.122571) (end 86.868 131.826) (width 0.7) (layer "B.Cu") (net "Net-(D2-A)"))
 (segment (start 68.9955 133.66525) (end 69.02675 133.66525) (width 0.7) (layer "B.Cu") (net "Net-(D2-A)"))
 (segment (start 86.868 131.826) (end 70.866 131.826) (width 0.7) (layer "B.Cu") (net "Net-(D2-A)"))
 (segment (start 68.9955 133.66525) (end 68.9955 135.77) (width 0.7) (layer "B.Cu") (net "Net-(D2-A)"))
 (segment (start 87.571429 130.08) (end 87.571429 131.122571) (width 0.7) (layer "B.Cu") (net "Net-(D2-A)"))
 (segment (start 69.02675 133.66525) (end 70.866 131.826) (width 0.7) (layer "B.Cu") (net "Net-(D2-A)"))
 (segment (start 153.38475 131.826) (end 155.00925 133.4505) (width 0.7) (layer "B.Cu") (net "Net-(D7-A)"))
 (segment (start 155.00925 133.4505) (end 155.00925 135.77) (width 0.7) (layer "B.Cu") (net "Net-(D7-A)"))
 (segment (start 100.428571 130.908571) (end 101.346 131.826) (width 0.7) (layer "B.Cu") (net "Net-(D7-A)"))
 (segment (start 145.542 131.826) (end 146.05 131.826) (width 0.7) (layer "B.Cu") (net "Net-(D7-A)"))
 (segment (start 100.428571 130.08) (end 100.428571 130.908571) (width 0.7) (layer "B.Cu") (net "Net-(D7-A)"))
 (segment (start 145.542 131.826) (end 153.38475 131.826) (width 0.7) (layer "B.Cu") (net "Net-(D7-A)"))
 (segment (start 101.346 131.826) (end 145.542 131.826) (width 0.7) (layer "B.Cu") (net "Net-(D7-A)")))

